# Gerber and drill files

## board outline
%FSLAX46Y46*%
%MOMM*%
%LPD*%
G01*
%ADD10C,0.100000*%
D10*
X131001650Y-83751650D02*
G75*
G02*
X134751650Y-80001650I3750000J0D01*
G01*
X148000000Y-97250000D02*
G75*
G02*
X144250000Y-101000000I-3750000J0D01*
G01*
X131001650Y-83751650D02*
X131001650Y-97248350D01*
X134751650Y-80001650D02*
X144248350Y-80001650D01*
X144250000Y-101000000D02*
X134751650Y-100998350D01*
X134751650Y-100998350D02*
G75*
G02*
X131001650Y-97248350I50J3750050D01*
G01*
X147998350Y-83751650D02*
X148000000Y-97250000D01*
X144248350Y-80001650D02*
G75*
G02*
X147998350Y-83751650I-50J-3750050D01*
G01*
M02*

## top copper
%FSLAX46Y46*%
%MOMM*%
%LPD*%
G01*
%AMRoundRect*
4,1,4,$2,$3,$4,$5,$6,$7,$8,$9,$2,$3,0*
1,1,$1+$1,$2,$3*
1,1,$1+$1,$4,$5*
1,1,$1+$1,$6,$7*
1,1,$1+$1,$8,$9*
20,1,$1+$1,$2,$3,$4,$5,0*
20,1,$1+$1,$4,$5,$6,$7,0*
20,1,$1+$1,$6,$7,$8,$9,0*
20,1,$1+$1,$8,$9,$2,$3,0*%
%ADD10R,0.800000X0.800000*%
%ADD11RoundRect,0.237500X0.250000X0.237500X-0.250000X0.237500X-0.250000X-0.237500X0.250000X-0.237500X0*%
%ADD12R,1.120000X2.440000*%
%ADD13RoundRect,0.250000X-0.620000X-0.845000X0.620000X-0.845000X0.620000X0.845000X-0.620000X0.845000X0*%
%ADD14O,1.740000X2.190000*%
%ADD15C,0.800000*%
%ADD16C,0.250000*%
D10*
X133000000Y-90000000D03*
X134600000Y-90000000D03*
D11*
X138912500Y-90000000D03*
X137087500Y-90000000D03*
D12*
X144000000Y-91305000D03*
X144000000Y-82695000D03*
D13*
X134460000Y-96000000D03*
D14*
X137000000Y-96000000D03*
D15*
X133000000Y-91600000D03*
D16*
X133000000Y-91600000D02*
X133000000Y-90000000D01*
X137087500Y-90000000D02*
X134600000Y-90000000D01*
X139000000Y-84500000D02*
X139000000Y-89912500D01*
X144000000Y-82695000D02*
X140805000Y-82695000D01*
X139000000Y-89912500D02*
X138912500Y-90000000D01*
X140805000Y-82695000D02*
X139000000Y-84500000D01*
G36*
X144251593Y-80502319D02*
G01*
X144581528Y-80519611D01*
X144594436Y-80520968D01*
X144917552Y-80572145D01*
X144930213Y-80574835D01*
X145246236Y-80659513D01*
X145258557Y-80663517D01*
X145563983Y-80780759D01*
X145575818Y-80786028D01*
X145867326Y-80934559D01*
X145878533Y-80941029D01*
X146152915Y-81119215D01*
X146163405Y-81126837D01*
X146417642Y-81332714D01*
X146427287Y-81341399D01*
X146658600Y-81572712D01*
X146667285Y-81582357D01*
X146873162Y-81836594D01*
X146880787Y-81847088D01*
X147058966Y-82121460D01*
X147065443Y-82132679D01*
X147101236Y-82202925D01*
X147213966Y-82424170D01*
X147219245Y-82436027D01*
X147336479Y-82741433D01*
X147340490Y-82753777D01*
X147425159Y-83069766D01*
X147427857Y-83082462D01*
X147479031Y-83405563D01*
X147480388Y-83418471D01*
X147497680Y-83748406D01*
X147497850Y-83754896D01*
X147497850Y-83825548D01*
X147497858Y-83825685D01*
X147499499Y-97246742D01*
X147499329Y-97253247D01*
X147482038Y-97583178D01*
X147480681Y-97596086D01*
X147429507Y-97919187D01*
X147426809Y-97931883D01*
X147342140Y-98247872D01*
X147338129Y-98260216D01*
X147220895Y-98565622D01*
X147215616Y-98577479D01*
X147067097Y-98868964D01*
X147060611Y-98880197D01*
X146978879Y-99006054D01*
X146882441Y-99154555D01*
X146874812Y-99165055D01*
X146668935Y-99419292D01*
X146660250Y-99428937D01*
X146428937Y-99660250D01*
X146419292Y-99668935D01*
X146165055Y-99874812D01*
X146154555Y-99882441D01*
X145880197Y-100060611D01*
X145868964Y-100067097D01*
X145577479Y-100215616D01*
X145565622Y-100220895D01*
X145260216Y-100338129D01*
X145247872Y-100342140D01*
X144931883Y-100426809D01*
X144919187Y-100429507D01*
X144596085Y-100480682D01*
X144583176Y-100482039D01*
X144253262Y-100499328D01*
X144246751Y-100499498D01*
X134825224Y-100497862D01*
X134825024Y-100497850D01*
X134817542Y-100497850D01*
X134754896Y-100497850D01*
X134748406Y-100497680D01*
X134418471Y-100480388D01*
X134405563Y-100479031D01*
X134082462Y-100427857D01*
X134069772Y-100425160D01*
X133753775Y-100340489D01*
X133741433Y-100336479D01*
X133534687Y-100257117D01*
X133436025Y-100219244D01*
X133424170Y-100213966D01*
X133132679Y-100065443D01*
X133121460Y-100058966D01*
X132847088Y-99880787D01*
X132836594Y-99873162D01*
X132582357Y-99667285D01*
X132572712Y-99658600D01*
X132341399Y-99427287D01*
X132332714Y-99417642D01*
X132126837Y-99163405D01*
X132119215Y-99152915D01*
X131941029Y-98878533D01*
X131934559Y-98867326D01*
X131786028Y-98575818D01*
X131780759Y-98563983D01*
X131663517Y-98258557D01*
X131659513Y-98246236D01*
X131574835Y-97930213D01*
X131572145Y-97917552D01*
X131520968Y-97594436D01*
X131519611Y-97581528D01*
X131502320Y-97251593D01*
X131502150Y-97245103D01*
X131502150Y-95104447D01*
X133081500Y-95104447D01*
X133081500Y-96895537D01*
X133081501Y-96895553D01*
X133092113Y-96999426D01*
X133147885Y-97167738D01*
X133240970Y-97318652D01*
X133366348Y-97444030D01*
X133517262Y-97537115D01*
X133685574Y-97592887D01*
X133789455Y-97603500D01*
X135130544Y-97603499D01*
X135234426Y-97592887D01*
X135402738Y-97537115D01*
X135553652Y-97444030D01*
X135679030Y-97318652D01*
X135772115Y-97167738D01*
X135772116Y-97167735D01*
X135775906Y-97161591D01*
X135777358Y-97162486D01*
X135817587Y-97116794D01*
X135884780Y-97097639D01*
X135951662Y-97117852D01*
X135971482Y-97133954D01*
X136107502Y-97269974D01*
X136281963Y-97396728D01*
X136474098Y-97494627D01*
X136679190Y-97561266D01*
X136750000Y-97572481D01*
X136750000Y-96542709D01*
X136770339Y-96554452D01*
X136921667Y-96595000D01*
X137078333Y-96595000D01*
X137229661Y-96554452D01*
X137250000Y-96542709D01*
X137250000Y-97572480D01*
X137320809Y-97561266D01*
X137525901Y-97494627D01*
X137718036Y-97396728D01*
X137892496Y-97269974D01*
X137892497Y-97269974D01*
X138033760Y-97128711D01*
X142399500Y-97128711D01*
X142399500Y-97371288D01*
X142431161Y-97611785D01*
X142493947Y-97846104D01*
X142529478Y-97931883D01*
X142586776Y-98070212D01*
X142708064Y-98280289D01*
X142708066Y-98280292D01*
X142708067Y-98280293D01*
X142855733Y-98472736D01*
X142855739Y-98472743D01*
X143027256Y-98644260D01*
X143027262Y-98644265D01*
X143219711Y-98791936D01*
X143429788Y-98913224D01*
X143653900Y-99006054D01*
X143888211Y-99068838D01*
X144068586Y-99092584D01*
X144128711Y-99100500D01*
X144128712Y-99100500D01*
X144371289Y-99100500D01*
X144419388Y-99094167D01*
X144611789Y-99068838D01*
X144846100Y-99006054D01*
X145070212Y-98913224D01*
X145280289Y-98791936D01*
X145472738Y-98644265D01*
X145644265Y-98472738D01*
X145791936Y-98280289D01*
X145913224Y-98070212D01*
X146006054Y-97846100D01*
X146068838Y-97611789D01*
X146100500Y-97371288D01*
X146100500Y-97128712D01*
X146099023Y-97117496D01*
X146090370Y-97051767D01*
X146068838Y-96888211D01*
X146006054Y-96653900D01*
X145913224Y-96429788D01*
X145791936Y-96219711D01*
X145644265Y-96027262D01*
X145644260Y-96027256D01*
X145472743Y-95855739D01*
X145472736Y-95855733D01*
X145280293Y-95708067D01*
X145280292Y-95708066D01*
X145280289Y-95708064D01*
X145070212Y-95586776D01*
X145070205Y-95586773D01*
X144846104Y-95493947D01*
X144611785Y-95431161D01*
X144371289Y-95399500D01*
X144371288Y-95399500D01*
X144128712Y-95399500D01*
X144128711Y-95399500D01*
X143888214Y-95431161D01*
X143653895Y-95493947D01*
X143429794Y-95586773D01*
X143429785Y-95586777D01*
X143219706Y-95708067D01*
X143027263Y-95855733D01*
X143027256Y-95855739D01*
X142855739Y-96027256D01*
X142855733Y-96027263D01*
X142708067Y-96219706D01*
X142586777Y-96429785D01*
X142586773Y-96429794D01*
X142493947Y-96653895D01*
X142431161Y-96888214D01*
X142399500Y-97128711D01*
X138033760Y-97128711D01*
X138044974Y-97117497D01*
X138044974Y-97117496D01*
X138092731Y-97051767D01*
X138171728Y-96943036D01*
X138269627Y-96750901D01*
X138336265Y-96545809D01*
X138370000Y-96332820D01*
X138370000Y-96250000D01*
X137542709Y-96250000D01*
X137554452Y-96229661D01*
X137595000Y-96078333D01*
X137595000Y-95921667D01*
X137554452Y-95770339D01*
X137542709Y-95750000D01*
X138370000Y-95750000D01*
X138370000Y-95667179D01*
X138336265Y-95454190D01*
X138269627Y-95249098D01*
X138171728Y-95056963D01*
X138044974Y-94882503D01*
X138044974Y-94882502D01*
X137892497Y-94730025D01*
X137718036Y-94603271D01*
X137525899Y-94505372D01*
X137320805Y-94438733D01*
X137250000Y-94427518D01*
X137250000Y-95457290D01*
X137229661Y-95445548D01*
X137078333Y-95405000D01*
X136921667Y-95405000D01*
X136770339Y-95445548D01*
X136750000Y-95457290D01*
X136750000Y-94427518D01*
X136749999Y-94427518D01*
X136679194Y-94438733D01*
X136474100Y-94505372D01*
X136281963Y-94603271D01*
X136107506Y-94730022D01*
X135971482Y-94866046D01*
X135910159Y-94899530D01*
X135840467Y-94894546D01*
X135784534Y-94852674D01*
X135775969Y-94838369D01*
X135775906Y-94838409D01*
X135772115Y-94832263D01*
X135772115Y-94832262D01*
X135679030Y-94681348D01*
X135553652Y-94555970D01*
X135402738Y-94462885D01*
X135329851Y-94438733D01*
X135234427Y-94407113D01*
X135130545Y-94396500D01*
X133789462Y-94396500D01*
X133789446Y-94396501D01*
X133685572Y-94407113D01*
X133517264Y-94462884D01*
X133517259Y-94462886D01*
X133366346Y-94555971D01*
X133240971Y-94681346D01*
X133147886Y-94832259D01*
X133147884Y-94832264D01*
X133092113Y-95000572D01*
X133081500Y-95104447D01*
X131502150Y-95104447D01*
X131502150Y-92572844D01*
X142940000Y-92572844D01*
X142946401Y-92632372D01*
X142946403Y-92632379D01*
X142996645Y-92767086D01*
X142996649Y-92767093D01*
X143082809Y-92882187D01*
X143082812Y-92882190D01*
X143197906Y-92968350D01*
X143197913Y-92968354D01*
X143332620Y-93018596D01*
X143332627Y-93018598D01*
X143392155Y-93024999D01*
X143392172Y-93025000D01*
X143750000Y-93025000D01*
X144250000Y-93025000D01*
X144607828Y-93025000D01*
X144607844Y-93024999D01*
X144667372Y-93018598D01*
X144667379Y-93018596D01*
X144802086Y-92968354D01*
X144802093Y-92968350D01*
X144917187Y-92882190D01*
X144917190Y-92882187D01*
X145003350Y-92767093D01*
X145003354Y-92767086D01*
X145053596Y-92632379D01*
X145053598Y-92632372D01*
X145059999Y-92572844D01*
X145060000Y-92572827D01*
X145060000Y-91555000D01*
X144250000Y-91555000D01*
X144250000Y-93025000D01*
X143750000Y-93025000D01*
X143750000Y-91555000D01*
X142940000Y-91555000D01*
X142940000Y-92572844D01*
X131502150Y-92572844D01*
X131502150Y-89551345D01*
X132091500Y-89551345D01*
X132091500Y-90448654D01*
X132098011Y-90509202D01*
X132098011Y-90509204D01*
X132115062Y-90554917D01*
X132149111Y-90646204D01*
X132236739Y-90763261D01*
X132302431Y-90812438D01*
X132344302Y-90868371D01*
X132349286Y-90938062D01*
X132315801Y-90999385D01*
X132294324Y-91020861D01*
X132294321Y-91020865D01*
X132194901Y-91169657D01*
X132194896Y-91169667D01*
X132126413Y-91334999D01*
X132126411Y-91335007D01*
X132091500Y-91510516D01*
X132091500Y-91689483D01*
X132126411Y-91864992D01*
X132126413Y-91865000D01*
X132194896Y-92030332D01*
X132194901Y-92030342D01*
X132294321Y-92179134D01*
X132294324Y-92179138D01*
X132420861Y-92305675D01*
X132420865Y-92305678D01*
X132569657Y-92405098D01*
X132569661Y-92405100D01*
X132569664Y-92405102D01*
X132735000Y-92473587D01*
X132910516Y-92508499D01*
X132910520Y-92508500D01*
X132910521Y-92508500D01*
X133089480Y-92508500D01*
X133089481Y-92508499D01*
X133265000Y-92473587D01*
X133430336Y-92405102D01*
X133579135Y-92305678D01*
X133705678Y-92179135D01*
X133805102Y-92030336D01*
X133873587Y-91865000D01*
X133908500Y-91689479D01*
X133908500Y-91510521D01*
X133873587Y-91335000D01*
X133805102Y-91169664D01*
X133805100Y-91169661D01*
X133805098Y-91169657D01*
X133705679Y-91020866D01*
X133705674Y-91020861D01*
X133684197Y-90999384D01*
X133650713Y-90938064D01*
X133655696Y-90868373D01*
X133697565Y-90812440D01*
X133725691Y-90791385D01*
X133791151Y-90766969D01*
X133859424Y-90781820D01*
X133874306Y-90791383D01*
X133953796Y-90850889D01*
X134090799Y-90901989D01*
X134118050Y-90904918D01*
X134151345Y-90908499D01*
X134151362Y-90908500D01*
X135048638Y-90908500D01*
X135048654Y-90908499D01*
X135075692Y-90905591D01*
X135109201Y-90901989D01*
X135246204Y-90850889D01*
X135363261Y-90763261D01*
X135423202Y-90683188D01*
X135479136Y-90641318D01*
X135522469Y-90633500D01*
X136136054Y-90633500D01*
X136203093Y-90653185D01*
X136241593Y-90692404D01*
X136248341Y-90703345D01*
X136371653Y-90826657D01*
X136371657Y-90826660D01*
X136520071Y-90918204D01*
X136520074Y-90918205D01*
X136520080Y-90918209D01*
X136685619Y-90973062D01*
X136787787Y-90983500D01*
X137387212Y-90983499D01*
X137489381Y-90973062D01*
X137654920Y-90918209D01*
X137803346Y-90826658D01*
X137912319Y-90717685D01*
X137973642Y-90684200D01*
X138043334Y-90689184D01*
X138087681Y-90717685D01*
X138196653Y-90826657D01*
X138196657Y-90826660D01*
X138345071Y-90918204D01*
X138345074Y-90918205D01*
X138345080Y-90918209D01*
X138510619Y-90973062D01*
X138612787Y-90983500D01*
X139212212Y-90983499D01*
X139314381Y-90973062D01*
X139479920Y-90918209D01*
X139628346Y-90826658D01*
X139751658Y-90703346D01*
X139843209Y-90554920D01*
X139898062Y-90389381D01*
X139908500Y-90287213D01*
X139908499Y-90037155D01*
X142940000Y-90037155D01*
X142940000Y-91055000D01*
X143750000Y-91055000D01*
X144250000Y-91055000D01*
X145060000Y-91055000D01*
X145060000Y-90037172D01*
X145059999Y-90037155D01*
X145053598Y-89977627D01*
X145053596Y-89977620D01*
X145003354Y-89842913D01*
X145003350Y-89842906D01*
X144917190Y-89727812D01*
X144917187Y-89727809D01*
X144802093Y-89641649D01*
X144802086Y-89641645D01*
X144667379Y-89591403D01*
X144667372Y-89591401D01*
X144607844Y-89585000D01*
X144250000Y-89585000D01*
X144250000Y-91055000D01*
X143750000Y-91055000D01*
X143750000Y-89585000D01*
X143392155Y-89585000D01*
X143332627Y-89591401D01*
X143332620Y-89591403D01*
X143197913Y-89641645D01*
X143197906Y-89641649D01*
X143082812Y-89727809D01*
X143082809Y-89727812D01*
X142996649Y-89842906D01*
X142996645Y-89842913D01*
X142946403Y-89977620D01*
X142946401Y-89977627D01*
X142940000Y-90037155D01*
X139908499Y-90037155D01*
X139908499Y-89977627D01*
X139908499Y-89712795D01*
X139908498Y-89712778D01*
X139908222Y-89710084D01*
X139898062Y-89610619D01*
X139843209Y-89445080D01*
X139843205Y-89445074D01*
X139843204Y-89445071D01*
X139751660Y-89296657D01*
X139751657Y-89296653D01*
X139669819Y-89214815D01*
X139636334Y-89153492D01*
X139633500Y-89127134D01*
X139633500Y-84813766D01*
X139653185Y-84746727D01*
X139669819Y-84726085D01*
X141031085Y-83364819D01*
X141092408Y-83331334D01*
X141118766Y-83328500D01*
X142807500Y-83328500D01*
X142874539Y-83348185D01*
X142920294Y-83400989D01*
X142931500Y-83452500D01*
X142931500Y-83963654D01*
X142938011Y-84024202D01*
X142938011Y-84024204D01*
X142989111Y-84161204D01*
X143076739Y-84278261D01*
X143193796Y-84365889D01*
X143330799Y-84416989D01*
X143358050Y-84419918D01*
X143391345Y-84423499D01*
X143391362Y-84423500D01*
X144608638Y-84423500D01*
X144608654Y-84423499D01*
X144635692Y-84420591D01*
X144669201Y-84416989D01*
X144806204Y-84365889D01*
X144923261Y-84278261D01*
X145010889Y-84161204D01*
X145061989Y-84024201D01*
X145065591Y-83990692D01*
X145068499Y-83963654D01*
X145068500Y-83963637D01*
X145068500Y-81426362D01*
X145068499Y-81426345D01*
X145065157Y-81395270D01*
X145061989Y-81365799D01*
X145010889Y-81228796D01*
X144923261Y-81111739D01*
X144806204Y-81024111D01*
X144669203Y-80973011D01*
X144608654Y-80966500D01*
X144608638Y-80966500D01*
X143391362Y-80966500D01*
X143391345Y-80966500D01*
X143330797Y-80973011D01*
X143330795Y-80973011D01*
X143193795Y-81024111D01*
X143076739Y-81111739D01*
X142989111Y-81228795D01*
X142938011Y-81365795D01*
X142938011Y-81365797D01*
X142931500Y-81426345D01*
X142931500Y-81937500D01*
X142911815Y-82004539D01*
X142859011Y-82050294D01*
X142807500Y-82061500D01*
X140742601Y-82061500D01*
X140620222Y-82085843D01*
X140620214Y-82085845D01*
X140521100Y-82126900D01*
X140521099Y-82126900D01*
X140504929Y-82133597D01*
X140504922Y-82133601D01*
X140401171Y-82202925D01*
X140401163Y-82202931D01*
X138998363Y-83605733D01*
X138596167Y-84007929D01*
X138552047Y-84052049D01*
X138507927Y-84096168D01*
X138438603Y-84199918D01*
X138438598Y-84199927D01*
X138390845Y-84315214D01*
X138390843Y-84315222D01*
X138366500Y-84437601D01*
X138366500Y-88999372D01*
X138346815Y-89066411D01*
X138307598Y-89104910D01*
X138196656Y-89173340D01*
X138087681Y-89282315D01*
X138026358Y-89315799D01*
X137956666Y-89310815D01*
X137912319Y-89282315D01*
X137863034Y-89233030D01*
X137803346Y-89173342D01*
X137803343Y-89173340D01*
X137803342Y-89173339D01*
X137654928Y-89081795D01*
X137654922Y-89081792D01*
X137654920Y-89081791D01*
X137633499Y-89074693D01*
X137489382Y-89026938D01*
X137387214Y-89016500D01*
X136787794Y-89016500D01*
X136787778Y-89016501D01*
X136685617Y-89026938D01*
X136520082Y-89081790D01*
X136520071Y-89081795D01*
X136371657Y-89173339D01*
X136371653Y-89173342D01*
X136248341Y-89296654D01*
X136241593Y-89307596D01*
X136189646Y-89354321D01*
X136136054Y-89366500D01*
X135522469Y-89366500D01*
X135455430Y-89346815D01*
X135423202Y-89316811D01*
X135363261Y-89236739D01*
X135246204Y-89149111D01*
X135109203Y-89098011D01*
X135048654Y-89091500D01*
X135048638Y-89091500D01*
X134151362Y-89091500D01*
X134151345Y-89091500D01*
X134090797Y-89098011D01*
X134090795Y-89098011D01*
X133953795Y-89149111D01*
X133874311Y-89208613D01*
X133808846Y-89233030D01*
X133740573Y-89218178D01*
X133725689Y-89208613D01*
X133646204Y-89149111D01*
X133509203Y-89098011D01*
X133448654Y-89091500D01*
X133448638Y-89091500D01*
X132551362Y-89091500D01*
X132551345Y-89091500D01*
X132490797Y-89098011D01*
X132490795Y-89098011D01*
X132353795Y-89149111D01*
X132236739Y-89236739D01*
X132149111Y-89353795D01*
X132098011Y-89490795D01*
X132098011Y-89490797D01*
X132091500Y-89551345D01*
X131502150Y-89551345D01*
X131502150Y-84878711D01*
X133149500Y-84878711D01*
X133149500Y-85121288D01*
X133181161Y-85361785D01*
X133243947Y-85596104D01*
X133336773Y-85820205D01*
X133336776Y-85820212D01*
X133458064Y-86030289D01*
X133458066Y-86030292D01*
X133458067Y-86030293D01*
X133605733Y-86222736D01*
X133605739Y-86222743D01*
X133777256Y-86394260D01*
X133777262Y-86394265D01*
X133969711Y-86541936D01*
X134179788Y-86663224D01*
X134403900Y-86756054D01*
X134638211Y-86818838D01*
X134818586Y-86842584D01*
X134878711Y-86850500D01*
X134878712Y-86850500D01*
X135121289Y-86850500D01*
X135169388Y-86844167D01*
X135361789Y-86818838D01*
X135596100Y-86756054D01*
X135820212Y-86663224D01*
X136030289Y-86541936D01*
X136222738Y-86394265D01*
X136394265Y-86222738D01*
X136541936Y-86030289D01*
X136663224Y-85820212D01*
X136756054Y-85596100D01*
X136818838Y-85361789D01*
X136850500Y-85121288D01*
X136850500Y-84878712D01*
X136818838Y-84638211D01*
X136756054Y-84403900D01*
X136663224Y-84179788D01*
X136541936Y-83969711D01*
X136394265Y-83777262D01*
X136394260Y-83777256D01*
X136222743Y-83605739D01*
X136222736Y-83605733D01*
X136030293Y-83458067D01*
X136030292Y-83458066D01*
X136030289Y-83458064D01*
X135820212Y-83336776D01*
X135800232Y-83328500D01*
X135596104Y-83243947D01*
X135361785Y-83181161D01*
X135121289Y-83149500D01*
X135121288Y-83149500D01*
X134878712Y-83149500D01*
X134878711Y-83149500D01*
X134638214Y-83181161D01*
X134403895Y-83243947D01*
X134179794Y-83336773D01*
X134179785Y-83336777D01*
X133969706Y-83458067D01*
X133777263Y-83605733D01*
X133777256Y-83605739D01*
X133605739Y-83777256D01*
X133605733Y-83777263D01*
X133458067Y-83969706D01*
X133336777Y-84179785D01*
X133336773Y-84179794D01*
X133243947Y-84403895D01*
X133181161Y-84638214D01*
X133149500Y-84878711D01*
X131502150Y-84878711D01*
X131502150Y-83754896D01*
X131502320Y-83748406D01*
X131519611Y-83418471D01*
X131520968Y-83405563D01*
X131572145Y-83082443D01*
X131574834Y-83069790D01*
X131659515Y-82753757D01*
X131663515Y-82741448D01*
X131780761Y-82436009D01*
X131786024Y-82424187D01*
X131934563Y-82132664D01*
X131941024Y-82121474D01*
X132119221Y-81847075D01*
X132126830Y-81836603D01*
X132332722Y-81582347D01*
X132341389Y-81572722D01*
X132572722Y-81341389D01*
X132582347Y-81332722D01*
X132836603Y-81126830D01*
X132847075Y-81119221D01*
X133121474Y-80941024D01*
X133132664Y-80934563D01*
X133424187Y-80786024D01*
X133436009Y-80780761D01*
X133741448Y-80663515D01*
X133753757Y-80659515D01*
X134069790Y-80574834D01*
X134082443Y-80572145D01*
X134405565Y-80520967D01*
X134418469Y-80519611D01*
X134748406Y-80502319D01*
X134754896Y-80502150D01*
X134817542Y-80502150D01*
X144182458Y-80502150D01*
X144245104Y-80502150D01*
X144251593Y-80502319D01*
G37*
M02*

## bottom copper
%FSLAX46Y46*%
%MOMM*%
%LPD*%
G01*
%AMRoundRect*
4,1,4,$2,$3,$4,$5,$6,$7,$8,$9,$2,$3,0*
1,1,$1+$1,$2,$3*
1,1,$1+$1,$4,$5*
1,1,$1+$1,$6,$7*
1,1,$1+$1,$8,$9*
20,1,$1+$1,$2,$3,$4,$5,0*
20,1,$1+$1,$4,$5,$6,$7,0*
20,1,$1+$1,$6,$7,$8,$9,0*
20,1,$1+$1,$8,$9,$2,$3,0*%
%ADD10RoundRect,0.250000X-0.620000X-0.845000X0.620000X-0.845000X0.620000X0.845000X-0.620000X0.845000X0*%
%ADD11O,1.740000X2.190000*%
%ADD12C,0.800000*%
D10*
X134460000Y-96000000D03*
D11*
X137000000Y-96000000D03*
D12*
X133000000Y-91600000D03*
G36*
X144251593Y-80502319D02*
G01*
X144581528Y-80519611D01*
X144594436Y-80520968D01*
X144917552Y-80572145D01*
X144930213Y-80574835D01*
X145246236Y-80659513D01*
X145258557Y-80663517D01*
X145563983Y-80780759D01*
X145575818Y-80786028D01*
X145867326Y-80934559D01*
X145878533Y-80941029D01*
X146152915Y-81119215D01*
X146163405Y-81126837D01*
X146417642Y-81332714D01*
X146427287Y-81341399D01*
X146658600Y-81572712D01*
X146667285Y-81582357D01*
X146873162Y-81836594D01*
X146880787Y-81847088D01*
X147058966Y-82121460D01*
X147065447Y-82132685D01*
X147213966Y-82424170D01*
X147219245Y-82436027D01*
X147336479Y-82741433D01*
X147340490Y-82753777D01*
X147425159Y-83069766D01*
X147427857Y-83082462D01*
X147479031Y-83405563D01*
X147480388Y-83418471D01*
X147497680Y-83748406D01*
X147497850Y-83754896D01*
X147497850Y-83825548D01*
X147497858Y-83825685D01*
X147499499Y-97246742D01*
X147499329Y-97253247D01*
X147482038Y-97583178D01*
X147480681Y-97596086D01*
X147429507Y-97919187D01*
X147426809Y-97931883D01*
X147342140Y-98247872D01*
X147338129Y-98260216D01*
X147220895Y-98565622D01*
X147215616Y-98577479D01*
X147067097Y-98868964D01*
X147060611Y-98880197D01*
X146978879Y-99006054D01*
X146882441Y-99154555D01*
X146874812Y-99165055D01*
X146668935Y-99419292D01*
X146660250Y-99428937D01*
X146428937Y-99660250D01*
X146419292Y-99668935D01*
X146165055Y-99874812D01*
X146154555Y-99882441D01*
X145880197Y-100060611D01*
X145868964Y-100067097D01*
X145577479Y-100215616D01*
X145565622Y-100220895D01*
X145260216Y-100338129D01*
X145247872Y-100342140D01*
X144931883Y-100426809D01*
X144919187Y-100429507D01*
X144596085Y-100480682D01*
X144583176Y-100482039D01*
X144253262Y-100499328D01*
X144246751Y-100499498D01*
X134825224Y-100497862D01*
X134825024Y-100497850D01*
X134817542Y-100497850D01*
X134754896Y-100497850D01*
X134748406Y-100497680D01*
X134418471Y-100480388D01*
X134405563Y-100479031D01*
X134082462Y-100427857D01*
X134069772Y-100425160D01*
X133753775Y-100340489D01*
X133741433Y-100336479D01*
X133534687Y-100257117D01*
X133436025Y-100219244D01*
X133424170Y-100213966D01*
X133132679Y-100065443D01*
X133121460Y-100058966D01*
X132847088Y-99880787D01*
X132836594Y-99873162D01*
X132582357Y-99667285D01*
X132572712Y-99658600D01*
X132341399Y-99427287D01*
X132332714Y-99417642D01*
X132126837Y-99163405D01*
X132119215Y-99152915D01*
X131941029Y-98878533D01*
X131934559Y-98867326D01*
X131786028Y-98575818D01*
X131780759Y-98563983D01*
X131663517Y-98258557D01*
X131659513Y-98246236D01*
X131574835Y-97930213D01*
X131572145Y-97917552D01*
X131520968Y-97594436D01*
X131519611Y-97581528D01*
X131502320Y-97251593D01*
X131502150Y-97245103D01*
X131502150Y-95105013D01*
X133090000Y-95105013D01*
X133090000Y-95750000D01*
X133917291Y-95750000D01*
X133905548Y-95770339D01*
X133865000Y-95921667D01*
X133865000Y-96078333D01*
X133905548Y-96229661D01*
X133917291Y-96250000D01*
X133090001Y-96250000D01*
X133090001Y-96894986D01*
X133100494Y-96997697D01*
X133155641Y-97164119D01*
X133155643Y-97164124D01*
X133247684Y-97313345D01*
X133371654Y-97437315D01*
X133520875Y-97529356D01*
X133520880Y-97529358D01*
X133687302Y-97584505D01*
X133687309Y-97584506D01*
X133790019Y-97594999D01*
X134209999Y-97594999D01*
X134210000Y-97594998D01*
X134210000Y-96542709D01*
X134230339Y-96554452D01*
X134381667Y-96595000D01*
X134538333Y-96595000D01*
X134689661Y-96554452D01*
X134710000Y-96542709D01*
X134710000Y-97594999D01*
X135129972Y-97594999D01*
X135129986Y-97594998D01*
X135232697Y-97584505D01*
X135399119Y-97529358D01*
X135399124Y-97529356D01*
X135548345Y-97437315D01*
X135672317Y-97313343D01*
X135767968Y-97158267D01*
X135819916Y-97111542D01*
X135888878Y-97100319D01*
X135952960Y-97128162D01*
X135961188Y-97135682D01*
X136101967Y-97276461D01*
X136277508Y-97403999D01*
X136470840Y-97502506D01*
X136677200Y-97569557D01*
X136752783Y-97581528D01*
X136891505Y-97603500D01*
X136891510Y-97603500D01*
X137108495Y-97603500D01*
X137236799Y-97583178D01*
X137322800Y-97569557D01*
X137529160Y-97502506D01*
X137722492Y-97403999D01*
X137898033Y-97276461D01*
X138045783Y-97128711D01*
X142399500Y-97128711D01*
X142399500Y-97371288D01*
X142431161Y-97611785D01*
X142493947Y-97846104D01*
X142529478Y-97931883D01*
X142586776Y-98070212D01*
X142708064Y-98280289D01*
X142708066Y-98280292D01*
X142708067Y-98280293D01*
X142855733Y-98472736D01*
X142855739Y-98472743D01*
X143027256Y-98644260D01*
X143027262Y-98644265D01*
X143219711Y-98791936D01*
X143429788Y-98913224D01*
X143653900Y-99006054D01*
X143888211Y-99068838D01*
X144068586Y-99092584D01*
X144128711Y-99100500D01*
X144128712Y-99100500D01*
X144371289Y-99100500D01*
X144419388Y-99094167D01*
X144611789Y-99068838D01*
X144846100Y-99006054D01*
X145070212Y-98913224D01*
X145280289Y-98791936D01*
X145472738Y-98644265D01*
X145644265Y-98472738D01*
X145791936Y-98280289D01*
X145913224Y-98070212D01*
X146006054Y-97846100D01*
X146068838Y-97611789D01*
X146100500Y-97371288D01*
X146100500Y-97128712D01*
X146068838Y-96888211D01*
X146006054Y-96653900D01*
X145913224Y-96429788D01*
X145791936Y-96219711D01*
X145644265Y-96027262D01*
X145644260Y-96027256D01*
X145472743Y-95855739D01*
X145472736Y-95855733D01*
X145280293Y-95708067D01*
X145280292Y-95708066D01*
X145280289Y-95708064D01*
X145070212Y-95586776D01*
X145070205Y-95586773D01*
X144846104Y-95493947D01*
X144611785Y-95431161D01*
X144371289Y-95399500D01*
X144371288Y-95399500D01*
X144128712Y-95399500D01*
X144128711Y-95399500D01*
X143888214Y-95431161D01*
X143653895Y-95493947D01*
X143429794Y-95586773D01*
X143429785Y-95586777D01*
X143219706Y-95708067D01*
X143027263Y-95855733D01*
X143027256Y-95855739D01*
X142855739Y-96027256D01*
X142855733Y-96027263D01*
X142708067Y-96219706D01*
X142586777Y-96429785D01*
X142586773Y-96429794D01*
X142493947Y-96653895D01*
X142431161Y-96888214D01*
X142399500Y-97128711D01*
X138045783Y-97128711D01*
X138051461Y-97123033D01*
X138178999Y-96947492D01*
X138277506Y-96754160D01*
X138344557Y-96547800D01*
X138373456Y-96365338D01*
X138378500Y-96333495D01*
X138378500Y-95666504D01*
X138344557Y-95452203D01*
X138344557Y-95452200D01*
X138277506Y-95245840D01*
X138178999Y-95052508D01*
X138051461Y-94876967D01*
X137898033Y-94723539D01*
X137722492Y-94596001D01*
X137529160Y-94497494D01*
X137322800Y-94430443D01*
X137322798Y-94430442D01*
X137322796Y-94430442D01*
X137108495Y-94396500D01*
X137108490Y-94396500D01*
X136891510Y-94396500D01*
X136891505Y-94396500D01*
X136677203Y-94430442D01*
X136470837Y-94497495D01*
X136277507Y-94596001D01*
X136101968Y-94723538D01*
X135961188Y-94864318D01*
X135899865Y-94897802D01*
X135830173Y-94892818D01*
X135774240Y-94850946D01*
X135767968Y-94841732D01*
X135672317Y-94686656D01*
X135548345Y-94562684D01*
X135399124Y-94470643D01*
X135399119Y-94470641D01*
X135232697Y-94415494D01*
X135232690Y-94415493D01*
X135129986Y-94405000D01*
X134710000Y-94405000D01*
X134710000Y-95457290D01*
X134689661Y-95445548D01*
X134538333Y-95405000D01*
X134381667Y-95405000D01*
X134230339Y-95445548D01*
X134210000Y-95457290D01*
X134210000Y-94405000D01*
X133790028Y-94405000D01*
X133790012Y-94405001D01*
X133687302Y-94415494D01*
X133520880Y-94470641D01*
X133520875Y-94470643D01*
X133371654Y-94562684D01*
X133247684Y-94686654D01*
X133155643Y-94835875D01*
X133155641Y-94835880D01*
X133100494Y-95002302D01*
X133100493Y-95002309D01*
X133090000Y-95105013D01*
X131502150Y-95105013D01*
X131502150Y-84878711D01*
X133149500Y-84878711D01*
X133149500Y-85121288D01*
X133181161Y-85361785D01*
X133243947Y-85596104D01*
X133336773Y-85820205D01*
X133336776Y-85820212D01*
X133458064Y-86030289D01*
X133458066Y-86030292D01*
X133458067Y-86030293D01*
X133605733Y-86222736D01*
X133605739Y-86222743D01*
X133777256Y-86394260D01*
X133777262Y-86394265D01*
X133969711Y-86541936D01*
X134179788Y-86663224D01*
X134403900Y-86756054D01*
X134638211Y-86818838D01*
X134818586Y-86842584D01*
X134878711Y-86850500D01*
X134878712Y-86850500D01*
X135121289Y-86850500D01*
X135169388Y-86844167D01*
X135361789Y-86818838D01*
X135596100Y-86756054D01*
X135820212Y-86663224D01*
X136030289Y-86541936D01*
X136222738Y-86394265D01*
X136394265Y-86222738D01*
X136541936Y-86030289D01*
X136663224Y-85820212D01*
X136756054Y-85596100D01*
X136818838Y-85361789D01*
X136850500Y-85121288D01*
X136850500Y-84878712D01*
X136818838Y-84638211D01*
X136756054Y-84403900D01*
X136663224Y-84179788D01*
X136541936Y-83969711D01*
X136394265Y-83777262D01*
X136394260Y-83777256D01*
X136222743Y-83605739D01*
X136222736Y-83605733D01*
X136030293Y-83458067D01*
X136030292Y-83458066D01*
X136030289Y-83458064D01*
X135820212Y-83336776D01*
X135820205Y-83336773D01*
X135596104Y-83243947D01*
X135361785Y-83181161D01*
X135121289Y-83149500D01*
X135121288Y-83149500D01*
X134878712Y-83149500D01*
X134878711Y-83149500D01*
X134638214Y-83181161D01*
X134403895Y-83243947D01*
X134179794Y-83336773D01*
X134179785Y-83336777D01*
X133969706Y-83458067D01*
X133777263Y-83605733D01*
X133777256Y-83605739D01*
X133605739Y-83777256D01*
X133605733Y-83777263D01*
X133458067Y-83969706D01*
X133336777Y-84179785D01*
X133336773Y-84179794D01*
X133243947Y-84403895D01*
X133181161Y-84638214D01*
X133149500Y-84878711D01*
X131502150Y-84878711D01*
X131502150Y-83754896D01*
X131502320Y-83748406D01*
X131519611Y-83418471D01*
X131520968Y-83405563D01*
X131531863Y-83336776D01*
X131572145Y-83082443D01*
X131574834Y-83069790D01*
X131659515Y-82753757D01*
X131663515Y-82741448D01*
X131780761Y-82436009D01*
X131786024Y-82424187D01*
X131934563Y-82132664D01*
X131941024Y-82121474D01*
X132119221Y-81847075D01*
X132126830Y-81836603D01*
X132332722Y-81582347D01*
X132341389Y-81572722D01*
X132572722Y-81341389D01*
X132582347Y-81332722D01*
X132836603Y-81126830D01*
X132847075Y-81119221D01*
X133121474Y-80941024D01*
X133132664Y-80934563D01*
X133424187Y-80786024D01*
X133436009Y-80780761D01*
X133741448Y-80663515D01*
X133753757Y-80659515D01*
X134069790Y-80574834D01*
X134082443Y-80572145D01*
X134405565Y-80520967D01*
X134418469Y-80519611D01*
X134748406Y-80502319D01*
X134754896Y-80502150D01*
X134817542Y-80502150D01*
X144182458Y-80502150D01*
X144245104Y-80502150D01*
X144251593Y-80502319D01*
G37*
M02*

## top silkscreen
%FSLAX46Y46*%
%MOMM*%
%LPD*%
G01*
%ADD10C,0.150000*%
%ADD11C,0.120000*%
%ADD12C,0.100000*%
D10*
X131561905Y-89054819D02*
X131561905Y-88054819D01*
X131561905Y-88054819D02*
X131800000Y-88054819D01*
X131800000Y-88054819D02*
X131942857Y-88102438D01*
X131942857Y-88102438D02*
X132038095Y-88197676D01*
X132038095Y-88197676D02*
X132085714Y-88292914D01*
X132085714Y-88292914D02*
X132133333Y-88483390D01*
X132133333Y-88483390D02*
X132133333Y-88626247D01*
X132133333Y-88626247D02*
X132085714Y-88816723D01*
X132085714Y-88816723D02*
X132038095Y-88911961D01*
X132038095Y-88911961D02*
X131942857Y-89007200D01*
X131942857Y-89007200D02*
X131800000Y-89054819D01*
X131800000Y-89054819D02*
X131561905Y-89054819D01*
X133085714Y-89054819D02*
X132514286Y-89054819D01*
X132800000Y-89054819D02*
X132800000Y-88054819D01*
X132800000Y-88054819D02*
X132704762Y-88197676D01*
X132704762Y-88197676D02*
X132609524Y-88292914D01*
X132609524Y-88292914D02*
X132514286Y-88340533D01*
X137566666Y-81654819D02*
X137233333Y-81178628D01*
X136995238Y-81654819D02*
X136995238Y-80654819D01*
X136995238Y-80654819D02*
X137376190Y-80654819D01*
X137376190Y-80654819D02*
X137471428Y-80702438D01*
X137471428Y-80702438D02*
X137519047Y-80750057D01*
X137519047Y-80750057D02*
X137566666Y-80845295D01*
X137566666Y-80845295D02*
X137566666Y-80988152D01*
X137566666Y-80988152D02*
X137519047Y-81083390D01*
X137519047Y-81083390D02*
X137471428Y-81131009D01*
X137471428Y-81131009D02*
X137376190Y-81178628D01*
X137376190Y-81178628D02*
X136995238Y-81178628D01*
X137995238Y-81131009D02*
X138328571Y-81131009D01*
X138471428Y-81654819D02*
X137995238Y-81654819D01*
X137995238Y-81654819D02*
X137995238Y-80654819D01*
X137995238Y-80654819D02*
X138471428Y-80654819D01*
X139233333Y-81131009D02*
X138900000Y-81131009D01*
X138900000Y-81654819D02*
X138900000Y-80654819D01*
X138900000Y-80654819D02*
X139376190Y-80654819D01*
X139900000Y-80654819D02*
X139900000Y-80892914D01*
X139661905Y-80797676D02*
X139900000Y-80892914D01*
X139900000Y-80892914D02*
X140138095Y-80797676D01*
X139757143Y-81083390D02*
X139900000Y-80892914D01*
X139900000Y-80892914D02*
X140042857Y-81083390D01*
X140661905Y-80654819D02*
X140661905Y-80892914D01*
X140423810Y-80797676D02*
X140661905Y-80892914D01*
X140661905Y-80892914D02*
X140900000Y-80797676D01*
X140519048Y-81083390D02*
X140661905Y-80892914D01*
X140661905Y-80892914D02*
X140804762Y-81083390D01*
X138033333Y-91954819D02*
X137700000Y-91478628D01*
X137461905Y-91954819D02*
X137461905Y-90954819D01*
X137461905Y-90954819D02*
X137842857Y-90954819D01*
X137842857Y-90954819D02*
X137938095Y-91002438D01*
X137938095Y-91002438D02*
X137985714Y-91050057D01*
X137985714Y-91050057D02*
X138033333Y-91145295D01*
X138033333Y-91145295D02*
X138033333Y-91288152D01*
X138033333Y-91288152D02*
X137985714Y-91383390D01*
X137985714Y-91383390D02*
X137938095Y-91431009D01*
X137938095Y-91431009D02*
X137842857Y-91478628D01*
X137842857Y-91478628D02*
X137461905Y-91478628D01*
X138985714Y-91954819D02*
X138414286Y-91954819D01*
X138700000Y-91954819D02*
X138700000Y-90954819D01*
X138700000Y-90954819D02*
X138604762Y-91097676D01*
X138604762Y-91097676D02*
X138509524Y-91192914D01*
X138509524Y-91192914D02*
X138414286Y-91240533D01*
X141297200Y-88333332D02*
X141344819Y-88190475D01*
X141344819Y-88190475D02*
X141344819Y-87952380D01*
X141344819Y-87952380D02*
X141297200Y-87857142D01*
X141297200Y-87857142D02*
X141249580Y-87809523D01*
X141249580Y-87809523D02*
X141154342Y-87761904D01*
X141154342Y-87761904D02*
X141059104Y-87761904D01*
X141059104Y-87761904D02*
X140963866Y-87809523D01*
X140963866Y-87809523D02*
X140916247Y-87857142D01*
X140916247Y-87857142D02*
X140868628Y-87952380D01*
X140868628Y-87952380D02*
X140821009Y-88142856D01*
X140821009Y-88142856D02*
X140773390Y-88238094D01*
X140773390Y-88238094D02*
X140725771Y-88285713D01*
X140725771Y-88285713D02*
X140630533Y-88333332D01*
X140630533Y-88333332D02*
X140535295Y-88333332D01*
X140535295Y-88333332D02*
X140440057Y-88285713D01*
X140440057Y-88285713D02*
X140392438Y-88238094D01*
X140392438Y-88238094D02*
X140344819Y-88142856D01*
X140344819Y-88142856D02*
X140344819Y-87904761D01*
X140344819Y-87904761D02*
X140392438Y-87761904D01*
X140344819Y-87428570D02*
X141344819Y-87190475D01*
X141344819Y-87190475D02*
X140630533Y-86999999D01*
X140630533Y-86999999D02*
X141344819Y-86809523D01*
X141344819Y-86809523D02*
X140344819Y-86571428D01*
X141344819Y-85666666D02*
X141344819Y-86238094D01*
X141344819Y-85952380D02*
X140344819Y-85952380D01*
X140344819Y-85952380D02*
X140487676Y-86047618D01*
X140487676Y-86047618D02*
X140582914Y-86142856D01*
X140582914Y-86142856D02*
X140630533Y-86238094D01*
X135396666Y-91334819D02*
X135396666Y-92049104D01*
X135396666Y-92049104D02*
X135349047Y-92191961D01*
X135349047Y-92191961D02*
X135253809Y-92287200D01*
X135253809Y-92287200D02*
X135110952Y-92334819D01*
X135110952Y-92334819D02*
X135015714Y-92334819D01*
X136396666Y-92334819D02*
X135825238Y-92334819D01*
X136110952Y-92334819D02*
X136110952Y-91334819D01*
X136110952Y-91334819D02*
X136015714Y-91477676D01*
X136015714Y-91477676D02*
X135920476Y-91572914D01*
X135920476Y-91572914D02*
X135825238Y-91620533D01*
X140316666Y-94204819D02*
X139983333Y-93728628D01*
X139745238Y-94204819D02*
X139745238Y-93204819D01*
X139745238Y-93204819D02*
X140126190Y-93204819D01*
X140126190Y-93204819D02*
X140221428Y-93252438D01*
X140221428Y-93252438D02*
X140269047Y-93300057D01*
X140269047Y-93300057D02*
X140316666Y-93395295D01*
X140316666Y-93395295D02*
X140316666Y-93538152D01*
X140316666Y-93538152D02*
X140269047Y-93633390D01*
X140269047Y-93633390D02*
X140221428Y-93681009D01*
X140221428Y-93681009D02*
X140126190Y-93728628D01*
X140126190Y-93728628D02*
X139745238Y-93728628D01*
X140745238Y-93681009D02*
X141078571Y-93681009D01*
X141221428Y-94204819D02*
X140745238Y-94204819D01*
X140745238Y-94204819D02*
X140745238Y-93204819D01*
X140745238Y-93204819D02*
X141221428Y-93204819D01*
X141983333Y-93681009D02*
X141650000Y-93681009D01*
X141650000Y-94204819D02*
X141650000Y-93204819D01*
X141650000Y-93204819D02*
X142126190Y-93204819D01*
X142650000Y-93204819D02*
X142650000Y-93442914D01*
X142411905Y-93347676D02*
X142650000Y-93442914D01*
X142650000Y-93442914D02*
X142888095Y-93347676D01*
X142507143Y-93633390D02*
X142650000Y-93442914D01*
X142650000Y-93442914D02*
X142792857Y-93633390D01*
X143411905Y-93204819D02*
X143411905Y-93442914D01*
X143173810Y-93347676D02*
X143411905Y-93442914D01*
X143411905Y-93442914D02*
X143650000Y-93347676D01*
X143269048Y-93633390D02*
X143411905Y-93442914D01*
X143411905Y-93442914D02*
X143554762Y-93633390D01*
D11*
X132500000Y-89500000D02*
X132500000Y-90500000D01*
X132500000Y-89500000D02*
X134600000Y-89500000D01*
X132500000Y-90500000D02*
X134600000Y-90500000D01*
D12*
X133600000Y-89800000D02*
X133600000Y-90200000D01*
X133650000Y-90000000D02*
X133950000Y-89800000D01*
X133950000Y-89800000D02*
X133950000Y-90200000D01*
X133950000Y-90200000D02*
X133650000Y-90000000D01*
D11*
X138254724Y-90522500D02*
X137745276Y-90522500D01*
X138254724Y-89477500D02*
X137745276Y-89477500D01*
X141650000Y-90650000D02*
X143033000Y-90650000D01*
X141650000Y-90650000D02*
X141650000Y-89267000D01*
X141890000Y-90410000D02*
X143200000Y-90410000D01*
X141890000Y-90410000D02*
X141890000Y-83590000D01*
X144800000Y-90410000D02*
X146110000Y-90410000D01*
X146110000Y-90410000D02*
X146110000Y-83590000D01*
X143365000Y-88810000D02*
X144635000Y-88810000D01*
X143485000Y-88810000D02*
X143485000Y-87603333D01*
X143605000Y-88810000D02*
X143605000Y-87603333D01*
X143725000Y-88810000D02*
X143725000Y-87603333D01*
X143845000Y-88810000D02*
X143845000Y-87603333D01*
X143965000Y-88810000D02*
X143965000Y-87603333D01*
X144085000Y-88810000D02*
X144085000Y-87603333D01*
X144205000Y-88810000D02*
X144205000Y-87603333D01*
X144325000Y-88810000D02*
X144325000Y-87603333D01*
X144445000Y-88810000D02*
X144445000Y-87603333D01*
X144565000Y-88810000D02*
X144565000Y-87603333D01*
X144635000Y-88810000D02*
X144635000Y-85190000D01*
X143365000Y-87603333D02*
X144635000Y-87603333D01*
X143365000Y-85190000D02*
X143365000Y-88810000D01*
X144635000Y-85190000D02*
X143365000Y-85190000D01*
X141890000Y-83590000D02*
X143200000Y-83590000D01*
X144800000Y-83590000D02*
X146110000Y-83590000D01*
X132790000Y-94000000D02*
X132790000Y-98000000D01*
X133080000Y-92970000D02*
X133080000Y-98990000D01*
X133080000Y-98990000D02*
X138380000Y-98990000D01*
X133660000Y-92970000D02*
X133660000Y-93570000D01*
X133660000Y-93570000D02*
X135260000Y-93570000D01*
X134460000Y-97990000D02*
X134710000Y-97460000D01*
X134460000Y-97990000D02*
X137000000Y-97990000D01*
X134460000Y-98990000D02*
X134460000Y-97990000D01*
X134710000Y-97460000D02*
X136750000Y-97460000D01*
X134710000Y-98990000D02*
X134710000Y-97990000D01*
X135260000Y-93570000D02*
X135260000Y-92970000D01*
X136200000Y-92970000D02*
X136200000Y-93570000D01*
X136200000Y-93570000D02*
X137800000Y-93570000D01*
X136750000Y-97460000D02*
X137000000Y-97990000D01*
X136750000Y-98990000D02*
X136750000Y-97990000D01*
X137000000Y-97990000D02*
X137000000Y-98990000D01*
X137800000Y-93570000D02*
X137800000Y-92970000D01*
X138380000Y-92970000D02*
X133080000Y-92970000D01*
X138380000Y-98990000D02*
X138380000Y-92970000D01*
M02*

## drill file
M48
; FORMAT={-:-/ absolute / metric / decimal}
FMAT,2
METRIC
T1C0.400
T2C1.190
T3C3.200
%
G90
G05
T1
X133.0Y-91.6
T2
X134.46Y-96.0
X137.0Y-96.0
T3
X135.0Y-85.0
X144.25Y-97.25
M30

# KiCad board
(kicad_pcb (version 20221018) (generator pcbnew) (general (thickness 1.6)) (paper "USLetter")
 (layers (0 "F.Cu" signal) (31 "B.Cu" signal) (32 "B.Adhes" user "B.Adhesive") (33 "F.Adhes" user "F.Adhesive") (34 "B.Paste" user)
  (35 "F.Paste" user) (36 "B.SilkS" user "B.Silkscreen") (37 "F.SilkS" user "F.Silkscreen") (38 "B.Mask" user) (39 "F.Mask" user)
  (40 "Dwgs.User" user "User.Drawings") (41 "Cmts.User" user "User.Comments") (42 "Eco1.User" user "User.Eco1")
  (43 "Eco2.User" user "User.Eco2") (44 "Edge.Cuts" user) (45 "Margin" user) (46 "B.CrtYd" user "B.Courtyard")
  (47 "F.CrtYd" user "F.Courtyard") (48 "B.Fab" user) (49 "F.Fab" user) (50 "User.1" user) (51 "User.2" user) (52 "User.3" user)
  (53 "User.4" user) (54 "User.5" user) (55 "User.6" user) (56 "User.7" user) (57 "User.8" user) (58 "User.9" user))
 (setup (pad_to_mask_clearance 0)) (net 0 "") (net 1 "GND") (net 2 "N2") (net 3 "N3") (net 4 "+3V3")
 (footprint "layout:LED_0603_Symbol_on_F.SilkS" (layer "F.Cu") (at 133.8 90)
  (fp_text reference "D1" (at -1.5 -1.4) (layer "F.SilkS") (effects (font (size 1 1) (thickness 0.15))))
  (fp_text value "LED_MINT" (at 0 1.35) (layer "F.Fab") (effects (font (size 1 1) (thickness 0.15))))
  (fp_line (start -1.3 -0.5) (end -1.3 0.5) (stroke (width 0.12) (type solid)) (layer "F.SilkS"))
  (fp_line (start -1.3 -0.5) (end 0.8 -0.5) (stroke (width 0.12) (type solid)) (layer "F.SilkS"))
  (fp_line (start -1.3 0.5) (end 0.8 0.5) (stroke (width 0.12) (type solid)) (layer "F.SilkS"))
  (fp_line (start -0.2 -0.2) (end -0.2 0.2) (stroke (width 0.1) (type solid)) (layer "F.SilkS"))
  (fp_line (start -0.15 0) (end 0.15 -0.2) (stroke (width 0.1) (type solid)) (layer "F.SilkS"))
  (fp_line (start 0.15 -0.2) (end 0.15 0.2) (stroke (width 0.1) (type solid)) (layer "F.SilkS"))
  (fp_line (start 0.15 0.2) (end -0.15 0) (stroke (width 0.1) (type solid)) (layer "F.SilkS"))
  (pad "1" smd rect (at -0.8 0 180) (size 0.8 0.8) (layers "F.Cu" "F.Paste" "F.Mask") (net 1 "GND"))
  (pad "2" smd rect (at 0.8 0 180) (size 0.8 0.8) (layers "F.Cu" "F.Paste" "F.Mask") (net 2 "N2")))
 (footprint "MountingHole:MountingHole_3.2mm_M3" (layer "F.Cu") (at 135 85)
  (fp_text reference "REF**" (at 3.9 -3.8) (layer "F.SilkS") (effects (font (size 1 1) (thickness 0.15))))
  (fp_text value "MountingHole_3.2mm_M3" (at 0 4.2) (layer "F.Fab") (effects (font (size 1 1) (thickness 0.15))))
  (pad "" np_thru_hole circle (at 0 0) (size 3.2 3.2) (drill 3.2) (layers "*.Cu" "*.Mask")))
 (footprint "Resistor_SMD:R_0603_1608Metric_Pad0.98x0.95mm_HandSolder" (layer "F.Cu") (at 138 90 180)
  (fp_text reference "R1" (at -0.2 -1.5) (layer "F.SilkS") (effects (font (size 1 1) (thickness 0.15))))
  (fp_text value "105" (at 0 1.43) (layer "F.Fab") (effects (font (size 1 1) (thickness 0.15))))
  (fp_line (start -0.254724 -0.5225) (end 0.254724 -0.5225) (stroke (width 0.12) (type solid)) (layer "F.SilkS"))
  (fp_line (start -0.254724 0.5225) (end 0.254724 0.5225) (stroke (width 0.12) (type solid)) (layer "F.SilkS"))
  (pad "1" smd roundrect (at -0.9125 0 180) (size 0.975 0.95) (layers "F.Cu" "F.Paste" "F.Mask") (roundrect_rratio 0.25) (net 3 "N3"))
  (pad "2" smd roundrect (at 0.9125 0 180) (size 0.975 0.95) (layers "F.Cu" "F.Paste" "F.Mask") (roundrect_rratio 0.25) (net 2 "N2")))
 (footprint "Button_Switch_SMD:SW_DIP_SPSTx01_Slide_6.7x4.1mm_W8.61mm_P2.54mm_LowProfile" (layer "F.Cu") (at 144 87 90)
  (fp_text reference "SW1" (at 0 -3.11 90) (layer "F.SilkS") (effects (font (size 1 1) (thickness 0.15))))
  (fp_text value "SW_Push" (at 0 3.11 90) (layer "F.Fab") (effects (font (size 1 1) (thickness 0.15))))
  (fp_line (start -3.65 -2.35) (end -3.65 -0.967) (stroke (width 0.12) (type solid)) (layer "F.SilkS"))
  (fp_line (start -3.65 -2.35) (end -2.267 -2.35) (stroke (width 0.12) (type solid)) (layer "F.SilkS"))
  (fp_line (start -3.41 -2.11) (end -3.41 -0.8) (stroke (width 0.12) (type solid)) (layer "F.SilkS"))
  (fp_line (start -3.41 -2.11) (end 3.41 -2.11) (stroke (width 0.12) (type solid)) (layer "F.SilkS"))
  (fp_line (start -3.41 0.8) (end -3.41 2.11) (stroke (width 0.12) (type solid)) (layer "F.SilkS"))
  (fp_line (start -3.41 2.11) (end 3.41 2.11) (stroke (width 0.12) (type solid)) (layer "F.SilkS"))
  (fp_line (start -1.81 -0.635) (end -1.81 0.635) (stroke (width 0.12) (type solid)) (layer "F.SilkS"))
  (fp_line (start -1.81 -0.515) (end -0.603333 -0.515) (stroke (width 0.12) (type solid)) (layer "F.SilkS"))
  (fp_line (start -1.81 -0.395) (end -0.603333 -0.395) (stroke (width 0.12) (type solid)) (layer "F.SilkS"))
  (fp_line (start -1.81 -0.275) (end -0.603333 -0.275) (stroke (width 0.12) (type solid)) (layer "F.SilkS"))
  (fp_line (start -1.81 -0.155) (end -0.603333 -0.155) (stroke (width 0.12) (type solid)) (layer "F.SilkS"))
  (fp_line (start -1.81 -0.035) (end -0.603333 -0.035) (stroke (width 0.12) (type solid)) (layer "F.SilkS"))
  (fp_line (start -1.81 0.085) (end -0.603333 0.085) (stroke (width 0.12) (type solid)) (layer "F.SilkS"))
  (fp_line (start -1.81 0.205) (end -0.603333 0.205) (stroke (width 0.12) (type solid)) (layer "F.SilkS"))
  (fp_line (start -1.81 0.325) (end -0.603333 0.325) (stroke (width 0.12) (type solid)) (layer "F.SilkS"))
  (fp_line (start -1.81 0.445) (end -0.603333 0.445) (stroke (width 0.12) (type solid)) (layer "F.SilkS"))
  (fp_line (start -1.81 0.565) (end -0.603333 0.565) (stroke (width 0.12) (type solid)) (layer "F.SilkS"))
  (fp_line (start -1.81 0.635) (end 1.81 0.635) (stroke (width 0.12) (type solid)) (layer "F.SilkS"))
  (fp_line (start -0.603333 -0.635) (end -0.603333 0.635) (stroke (width 0.12) (type solid)) (layer "F.SilkS"))
  (fp_line (start 1.81 -0.635) (end -1.81 -0.635) (stroke (width 0.12) (type solid)) (layer "F.SilkS"))
  (fp_line (start 1.81 0.635) (end 1.81 -0.635) (stroke (width 0.12) (type solid)) (layer "F.SilkS"))
  (fp_line (start 3.41 -2.11) (end 3.41 -0.8) (stroke (width 0.12) (type solid)) (layer "F.SilkS"))
  (fp_line (start 3.41 0.8) (end 3.41 2.11) (stroke (width 0.12) (type solid)) (layer "F.SilkS"))
  (pad "1" smd rect (at -4.305 0 90) (size 2.44 1.12) (layers "F.Cu" "F.Paste" "F.Mask") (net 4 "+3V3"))
  (pad "2" smd rect (at 4.305 0 90) (size 2.44 1.12) (layers "F.Cu" "F.Paste" "F.Mask") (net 3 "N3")))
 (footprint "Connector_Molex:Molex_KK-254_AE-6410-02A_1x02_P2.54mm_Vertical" (layer "F.Cu") (at 134.46 96)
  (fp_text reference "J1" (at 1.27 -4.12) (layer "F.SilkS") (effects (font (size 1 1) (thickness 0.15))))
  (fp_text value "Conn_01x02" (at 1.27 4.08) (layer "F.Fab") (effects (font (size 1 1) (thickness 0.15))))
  (fp_line (start -1.67 -2) (end -1.67 2) (stroke (width 0.12) (type solid)) (layer "F.SilkS"))
  (fp_line (start -1.38 -3.03) (end -1.38 2.99) (stroke (width 0.12) (type solid)) (layer "F.SilkS"))
  (fp_line (start -1.38 2.99) (end 3.92 2.99) (stroke (width 0.12) (type solid)) (layer "F.SilkS"))
  (fp_line (start -0.8 -3.03) (end -0.8 -2.43) (stroke (width 0.12) (type solid)) (layer "F.SilkS"))
  (fp_line (start -0.8 -2.43) (end 0.8 -2.43) (stroke (width 0.12) (type solid)) (layer "F.SilkS"))
  (fp_line (start 0 1.99) (end 0.25 1.46) (stroke (width 0.12) (type solid)) (layer "F.SilkS"))
  (fp_line (start 0 1.99) (end 2.54 1.99) (stroke (width 0.12) (type solid)) (layer "F.SilkS"))
  (fp_line (start 0 2.99) (end 0 1.99) (stroke (width 0.12) (type solid)) (layer "F.SilkS"))
  (fp_line (start 0.25 1.46) (end 2.29 1.46) (stroke (width 0.12) (type solid)) (layer "F.SilkS"))
  (fp_line (start 0.25 2.99) (end 0.25 1.99) (stroke (width 0.12) (type solid)) (layer "F.SilkS"))
  (fp_line (start 0.8 -2.43) (end 0.8 -3.03) (stroke (width 0.12) (type solid)) (layer "F.SilkS"))
  (fp_line (start 1.74 -3.03) (end 1.74 -2.43) (stroke (width 0.12) (type solid)) (layer "F.SilkS"))
  (fp_line (start 1.74 -2.43) (end 3.34 -2.43) (stroke (width 0.12) (type solid)) (layer "F.SilkS"))
  (fp_line (start 2.29 1.46) (end 2.54 1.99) (stroke (width 0.12) (type solid)) (layer "F.SilkS"))
  (fp_line (start 2.29 2.99) (end 2.29 1.99) (stroke (width 0.12) (type solid)) (layer "F.SilkS"))
  (fp_line (start 2.54 1.99) (end 2.54 2.99) (stroke (width 0.12) (type solid)) (layer "F.SilkS"))
  (fp_line (start 3.34 -2.43) (end 3.34 -3.03) (stroke (width 0.12) (type solid)) (layer "F.SilkS"))
  (fp_line (start 3.92 -3.03) (end -1.38 -3.03) (stroke (width 0.12) (type solid)) (layer "F.SilkS"))
  (fp_line (start 3.92 2.99) (end 3.92 -3.03) (stroke (width 0.12) (type solid)) (layer "F.SilkS"))
  (pad "1" thru_hole roundrect (at 0 0) (size 1.74 2.19) (drill 1.19) (layers "*.Cu" "*.Mask") (roundrect_rratio 0.143678) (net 1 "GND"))
  (pad "2" thru_hole oval (at 2.54 0) (size 1.74 2.19) (drill 1.19) (layers "*.Cu" "*.Mask") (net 4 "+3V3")))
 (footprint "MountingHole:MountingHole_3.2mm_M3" (layer "F.Cu") (at 144.25 97.25)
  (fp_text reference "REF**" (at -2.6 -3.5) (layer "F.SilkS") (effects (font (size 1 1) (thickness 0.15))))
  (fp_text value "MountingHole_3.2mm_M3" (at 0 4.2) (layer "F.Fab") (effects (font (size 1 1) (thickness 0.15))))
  (pad "" np_thru_hole circle (at 0 0) (size 3.2 3.2) (drill 3.2) (layers "F&B.Cu" "*.Mask")))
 (gr_arc (start 131.00165 83.75165) (mid 132.1 81.1) (end 134.75165 80.00165) (stroke (width 0.1) (type default)) (layer "Edge.Cuts"))
 (gr_arc (start 148 97.25) (mid 146.90165 99.90165) (end 144.25 101) (stroke (width 0.1) (type default)) (layer "Edge.Cuts"))
 (gr_line (start 131.00165 83.75165) (end 131.00165 97.24835) (stroke (width 0.1) (type default)) (layer "Edge.Cuts"))
 (gr_line (start 134.75165 80.00165) (end 144.24835 80.00165) (stroke (width 0.1) (type default)) (layer "Edge.Cuts"))
 (gr_line (start 144.25 101) (end 134.75165 100.99835) (stroke (width 0.1) (type default)) (layer "Edge.Cuts"))
 (gr_arc (start 134.75165 100.99835) (mid 132.1 99.9) (end 131.00165 97.24835) (stroke (width 0.1) (type default)) (layer "Edge.Cuts"))
 (gr_line (start 147.99835 83.75165) (end 148 97.25) (stroke (width 0.1) (type default)) (layer "Edge.Cuts"))
 (gr_arc (start 144.24835 80.00165) (mid 146.9 81.1) (end 147.99835 83.75165) (stroke (width 0.1) (type default)) (layer "Edge.Cuts"))
 (segment (start 133 91.6) (end 133 90) (width 0.25) (layer "F.Cu") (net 1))
 (via (at 133 91.6) (size 0.8) (drill 0.4) (layers "F.Cu" "B.Cu") (free) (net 1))
 (segment (start 137.0875 90) (end 134.6 90) (width 0.25) (layer "F.Cu") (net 2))
 (segment (start 139 84.5) (end 139 89.9125) (width 0.25) (layer "F.Cu") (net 3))
 (segment (start 144 82.695) (end 140.805 82.695) (width 0.25) (layer "F.Cu") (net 3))
 (segment (start 139 89.9125) (end 138.9125 90) (width 0.25) (layer "F.Cu") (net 3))
 (segment (start 140.805 82.695) (end 139 84.5) (width 0.25) (layer "F.Cu") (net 3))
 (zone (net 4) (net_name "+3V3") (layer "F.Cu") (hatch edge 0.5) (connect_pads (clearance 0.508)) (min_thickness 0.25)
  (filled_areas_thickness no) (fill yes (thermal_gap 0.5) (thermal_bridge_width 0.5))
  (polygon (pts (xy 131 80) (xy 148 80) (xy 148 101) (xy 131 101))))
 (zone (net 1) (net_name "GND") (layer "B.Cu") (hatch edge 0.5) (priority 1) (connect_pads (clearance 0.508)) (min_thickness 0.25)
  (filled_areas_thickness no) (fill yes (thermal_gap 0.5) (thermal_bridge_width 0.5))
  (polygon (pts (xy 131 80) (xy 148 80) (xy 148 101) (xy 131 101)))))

